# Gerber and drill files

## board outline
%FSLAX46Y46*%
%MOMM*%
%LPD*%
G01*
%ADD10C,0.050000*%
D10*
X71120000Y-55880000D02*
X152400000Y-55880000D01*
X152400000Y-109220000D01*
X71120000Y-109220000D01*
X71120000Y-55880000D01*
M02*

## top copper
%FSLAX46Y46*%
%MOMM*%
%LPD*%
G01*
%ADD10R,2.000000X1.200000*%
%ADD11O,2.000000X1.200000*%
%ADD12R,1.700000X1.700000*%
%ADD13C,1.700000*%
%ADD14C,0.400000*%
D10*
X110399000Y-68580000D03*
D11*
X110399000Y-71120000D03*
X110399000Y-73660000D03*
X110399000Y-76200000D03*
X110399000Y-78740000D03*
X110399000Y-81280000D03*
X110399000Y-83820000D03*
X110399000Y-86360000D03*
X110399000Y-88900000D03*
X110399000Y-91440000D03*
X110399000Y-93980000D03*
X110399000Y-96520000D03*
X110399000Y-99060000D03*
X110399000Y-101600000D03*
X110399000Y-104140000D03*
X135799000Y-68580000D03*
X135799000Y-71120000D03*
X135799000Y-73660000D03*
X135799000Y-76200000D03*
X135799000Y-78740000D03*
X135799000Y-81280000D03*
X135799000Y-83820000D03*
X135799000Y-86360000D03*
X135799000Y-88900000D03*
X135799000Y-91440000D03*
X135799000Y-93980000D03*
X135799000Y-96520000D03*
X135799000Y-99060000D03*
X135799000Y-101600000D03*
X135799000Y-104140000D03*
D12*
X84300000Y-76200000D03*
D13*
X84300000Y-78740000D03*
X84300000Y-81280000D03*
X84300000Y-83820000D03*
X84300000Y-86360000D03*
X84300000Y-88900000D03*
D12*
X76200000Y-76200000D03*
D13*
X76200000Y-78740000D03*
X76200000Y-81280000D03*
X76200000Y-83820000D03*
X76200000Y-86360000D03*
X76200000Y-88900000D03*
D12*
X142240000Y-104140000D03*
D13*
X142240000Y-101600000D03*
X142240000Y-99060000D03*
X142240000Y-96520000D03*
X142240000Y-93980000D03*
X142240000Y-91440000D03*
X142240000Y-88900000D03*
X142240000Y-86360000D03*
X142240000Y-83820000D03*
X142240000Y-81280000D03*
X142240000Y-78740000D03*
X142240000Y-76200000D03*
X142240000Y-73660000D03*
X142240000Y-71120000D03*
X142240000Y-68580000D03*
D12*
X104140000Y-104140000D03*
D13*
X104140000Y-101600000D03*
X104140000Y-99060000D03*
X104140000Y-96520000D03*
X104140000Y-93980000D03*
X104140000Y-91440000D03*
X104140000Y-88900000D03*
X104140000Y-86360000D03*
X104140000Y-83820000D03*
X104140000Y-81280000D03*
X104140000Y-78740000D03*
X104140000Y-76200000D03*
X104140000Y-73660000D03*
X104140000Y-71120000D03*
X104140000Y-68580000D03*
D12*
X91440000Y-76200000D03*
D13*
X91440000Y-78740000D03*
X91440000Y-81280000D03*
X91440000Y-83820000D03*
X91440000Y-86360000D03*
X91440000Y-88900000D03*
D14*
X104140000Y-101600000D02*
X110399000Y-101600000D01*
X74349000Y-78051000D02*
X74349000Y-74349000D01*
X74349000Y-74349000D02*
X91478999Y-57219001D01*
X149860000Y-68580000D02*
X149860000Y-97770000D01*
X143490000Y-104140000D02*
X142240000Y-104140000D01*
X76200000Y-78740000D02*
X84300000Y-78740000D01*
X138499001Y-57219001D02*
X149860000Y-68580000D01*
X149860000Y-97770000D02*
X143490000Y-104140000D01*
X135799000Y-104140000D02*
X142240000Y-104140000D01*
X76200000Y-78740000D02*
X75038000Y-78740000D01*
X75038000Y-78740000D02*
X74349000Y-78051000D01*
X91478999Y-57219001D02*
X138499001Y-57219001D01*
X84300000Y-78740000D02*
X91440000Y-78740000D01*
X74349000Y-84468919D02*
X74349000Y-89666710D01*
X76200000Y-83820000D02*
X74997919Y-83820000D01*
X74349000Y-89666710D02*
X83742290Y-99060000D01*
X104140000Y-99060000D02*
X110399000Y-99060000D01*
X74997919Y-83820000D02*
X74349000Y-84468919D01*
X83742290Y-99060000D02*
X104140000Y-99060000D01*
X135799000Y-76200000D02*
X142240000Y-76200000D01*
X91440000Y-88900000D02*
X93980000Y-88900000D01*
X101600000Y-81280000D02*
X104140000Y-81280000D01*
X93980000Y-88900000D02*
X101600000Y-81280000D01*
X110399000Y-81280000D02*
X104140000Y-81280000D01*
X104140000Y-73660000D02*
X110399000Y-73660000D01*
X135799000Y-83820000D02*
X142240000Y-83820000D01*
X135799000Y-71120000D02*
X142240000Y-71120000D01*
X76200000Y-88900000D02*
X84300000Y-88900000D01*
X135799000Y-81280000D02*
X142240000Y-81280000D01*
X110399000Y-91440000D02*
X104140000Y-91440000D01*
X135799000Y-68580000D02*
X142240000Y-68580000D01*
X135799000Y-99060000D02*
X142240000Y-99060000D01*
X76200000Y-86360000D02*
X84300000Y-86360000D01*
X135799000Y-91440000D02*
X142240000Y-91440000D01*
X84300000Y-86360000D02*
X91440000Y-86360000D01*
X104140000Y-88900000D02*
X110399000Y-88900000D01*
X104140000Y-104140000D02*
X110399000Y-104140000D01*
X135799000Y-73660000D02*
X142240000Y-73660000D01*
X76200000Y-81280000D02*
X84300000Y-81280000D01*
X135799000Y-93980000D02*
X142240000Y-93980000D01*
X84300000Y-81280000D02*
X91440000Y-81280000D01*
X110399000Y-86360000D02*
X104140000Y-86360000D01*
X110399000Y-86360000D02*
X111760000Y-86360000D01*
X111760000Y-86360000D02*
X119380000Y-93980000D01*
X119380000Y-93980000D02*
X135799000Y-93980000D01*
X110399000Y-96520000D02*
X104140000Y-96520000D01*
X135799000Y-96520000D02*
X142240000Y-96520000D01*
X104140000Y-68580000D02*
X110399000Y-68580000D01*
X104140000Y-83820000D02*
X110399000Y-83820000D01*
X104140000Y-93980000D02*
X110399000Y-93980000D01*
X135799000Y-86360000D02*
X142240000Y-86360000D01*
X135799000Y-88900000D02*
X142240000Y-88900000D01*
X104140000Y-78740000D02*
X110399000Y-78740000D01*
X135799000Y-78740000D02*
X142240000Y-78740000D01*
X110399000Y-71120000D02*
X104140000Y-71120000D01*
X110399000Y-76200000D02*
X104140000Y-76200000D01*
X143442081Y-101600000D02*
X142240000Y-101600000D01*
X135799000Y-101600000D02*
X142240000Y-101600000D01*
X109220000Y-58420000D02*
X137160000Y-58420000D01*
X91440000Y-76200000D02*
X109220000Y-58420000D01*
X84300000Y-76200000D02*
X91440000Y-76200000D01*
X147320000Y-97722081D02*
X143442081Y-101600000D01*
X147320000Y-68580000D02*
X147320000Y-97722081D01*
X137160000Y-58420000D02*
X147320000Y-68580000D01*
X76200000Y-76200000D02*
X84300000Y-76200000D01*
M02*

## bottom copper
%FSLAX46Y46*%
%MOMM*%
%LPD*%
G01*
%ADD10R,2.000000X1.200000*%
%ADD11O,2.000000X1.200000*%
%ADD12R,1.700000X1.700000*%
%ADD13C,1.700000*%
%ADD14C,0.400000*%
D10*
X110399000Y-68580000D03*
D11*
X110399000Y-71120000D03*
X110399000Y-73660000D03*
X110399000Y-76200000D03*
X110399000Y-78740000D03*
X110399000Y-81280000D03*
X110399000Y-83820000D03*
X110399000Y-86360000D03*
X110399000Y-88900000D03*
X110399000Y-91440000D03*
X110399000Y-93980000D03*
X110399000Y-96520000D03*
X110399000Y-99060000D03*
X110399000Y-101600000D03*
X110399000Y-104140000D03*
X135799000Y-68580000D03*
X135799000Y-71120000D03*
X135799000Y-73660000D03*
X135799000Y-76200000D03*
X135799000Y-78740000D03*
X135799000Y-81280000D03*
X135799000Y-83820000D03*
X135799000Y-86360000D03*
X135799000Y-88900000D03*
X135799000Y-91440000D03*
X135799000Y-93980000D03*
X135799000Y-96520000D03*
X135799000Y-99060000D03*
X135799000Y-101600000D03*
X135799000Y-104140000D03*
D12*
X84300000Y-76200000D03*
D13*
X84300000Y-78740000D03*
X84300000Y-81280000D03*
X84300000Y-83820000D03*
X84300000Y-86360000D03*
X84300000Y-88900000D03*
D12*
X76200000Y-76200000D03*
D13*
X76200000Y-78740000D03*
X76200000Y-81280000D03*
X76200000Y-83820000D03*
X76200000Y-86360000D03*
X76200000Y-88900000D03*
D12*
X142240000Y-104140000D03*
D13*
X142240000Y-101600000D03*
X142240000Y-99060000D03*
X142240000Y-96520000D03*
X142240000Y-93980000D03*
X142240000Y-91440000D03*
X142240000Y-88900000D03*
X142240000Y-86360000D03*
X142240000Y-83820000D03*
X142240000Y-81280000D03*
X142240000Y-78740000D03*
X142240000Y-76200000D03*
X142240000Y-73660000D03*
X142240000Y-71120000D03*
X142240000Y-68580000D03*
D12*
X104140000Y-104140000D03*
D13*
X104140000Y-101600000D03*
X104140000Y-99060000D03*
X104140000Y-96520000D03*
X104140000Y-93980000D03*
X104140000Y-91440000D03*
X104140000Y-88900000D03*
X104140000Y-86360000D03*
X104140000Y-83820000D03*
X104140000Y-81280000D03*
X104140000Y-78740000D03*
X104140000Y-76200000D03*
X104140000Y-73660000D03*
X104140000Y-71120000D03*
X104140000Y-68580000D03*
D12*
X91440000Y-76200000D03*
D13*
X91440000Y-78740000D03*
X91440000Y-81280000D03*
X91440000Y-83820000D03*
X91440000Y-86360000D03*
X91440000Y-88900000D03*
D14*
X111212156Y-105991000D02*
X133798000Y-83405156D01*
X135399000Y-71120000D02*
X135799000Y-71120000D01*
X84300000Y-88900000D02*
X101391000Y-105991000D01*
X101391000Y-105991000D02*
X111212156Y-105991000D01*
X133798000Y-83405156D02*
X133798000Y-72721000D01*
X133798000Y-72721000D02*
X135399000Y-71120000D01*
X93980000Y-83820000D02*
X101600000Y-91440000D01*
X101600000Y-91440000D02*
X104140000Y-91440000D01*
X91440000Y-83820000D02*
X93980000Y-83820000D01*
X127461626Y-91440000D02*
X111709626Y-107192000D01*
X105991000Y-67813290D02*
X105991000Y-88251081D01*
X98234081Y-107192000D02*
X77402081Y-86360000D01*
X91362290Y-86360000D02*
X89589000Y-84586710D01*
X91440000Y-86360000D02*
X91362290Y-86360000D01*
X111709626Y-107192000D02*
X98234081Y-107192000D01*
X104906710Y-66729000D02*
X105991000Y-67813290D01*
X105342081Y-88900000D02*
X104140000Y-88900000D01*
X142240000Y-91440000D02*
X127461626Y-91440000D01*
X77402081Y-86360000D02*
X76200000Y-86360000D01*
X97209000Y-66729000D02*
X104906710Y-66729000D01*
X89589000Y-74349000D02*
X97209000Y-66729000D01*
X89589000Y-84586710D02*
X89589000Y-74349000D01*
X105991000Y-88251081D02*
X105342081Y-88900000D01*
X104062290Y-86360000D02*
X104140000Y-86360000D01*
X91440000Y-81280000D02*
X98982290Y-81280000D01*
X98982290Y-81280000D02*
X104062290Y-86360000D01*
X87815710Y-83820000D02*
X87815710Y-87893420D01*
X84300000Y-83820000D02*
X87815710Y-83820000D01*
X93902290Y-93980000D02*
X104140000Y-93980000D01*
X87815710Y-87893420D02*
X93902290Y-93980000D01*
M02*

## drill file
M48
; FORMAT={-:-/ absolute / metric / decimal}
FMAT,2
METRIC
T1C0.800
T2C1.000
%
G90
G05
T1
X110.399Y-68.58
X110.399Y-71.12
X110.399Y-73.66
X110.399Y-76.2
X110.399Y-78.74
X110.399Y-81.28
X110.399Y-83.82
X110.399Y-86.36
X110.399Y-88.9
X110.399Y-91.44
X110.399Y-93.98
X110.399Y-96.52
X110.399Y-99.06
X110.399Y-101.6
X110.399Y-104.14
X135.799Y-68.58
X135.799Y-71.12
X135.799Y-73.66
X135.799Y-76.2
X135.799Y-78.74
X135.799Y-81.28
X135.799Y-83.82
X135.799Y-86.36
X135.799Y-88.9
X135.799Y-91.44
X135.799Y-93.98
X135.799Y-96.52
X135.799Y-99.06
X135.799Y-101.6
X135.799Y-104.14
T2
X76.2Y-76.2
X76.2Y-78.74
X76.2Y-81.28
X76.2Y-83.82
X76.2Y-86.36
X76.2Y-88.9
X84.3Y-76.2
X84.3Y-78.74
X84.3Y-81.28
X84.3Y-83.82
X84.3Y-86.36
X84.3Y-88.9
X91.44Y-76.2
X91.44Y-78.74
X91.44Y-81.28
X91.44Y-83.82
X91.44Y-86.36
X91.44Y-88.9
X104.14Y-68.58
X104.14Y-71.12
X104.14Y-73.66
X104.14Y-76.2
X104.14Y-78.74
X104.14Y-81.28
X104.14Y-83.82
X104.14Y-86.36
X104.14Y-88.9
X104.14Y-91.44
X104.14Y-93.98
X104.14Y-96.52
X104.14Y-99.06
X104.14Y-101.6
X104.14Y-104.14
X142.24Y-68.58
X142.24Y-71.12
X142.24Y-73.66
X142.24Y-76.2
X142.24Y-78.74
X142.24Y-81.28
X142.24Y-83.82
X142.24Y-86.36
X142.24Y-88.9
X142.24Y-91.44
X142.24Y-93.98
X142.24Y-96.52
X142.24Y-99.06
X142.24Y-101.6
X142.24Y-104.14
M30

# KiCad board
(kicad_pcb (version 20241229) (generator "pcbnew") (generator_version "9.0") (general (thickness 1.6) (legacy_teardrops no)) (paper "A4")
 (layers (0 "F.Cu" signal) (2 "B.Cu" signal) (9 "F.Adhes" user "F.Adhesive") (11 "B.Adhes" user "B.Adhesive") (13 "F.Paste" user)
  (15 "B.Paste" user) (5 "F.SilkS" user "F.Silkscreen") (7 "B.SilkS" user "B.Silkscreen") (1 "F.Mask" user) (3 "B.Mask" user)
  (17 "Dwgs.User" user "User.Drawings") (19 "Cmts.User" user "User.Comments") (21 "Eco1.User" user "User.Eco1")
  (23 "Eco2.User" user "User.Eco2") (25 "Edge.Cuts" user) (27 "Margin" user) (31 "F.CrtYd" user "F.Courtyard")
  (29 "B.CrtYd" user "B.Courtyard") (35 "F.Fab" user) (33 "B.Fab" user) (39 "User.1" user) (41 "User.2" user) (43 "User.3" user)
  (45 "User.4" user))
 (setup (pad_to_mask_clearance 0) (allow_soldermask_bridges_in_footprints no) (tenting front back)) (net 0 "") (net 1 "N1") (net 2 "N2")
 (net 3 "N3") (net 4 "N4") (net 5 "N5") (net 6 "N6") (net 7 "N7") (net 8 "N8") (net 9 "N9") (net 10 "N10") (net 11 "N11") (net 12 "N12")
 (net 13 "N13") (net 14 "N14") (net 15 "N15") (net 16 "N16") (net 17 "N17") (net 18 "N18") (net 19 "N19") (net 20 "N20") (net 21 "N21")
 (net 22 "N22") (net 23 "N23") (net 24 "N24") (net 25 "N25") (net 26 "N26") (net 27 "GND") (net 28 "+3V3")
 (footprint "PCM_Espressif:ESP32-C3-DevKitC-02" (layer "F.Cu") (at 110.399 68.58)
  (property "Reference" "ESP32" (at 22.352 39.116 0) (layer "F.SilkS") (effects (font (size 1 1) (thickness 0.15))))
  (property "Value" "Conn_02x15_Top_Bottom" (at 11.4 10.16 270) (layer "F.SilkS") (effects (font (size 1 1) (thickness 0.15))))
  (pad "1" thru_hole rect (at 0 0 270) (size 1.2 2) (drill 0.8) (layers "*.Cu" "*.Mask") (remove_unused_layers no) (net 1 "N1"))
  (pad "2" thru_hole oval (at 0 2.54 270) (size 1.2 2) (drill 0.8) (layers "*.Cu" "*.Mask") (remove_unused_layers no) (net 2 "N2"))
  (pad "3" thru_hole oval (at 0 5.08 270) (size 1.2 2) (drill 0.8) (layers "*.Cu" "*.Mask") (remove_unused_layers no) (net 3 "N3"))
  (pad "4" thru_hole oval (at 0 7.62 270) (size 1.2 2) (drill 0.8) (layers "*.Cu" "*.Mask") (remove_unused_layers no) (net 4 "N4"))
  (pad "5" thru_hole oval (at 0 10.16 270) (size 1.2 2) (drill 0.8) (layers "*.Cu" "*.Mask") (remove_unused_layers no) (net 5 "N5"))
  (pad "6" thru_hole oval (at 0 12.7 270) (size 1.2 2) (drill 0.8) (layers "*.Cu" "*.Mask") (remove_unused_layers no) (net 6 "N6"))
  (pad "7" thru_hole oval (at 0 15.24 270) (size 1.2 2) (drill 0.8) (layers "*.Cu" "*.Mask") (remove_unused_layers no) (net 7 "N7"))
  (pad "8" thru_hole oval (at 0 17.78 270) (size 1.2 2) (drill 0.8) (layers "*.Cu" "*.Mask") (remove_unused_layers no) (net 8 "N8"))
  (pad "9" thru_hole oval (at 0 20.32 270) (size 1.2 2) (drill 0.8) (layers "*.Cu" "*.Mask") (remove_unused_layers no) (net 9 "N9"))
  (pad "10" thru_hole oval (at 0 22.86 270) (size 1.2 2) (drill 0.8) (layers "*.Cu" "*.Mask") (remove_unused_layers no) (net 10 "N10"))
  (pad "11" thru_hole oval (at 0 25.4 270) (size 1.2 2) (drill 0.8) (layers "*.Cu" "*.Mask") (remove_unused_layers no) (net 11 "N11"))
  (pad "12" thru_hole oval (at 0 27.94 270) (size 1.2 2) (drill 0.8) (layers "*.Cu" "*.Mask") (remove_unused_layers no) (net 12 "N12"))
  (pad "13" thru_hole oval (at 0 30.48 270) (size 1.2 2) (drill 0.8) (layers "*.Cu" "*.Mask") (remove_unused_layers no) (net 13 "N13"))
  (pad "14" thru_hole oval (at 0 33.02 270) (size 1.2 2) (drill 0.8) (layers "*.Cu" "*.Mask") (remove_unused_layers no) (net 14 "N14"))
  (pad "15" thru_hole oval (at 0 35.56 270) (size 1.2 2) (drill 0.8) (layers "*.Cu" "*.Mask") (remove_unused_layers no) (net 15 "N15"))
  (pad "16" thru_hole oval (at 25.4 0 90) (size 1.2 2) (drill 0.8) (layers "*.Cu" "*.Mask") (remove_unused_layers no) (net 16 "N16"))
  (pad "17" thru_hole oval (at 25.4 2.54 90) (size 1.2 2) (drill 0.8) (layers "*.Cu" "*.Mask") (remove_unused_layers no) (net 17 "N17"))
  (pad "18" thru_hole oval (at 25.4 5.08 90) (size 1.2 2) (drill 0.8) (layers "*.Cu" "*.Mask") (remove_unused_layers no) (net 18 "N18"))
  (pad "19" thru_hole oval (at 25.4 7.62 90) (size 1.2 2) (drill 0.8) (layers "*.Cu" "*.Mask") (remove_unused_layers no) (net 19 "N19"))
  (pad "20" thru_hole oval (at 25.4 10.16 90) (size 1.2 2) (drill 0.8) (layers "*.Cu" "*.Mask") (remove_unused_layers no) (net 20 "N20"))
  (pad "21" thru_hole oval (at 25.4 12.7 90) (size 1.2 2) (drill 0.8) (layers "*.Cu" "*.Mask") (remove_unused_layers no) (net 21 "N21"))
  (pad "22" thru_hole oval (at 25.4 15.24 90) (size 1.2 2) (drill 0.8) (layers "*.Cu" "*.Mask") (remove_unused_layers no) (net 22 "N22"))
  (pad "23" thru_hole oval (at 25.4 17.78 90) (size 1.2 2) (drill 0.8) (layers "*.Cu" "*.Mask") (remove_unused_layers no) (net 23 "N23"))
  (pad "24" thru_hole oval (at 25.4 20.32 90) (size 1.2 2) (drill 0.8) (layers "*.Cu" "*.Mask") (remove_unused_layers no) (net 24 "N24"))
  (pad "25" thru_hole oval (at 25.4 22.86 90) (size 1.2 2) (drill 0.8) (layers "*.Cu" "*.Mask") (remove_unused_layers no) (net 9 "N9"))
  (pad "26" thru_hole oval (at 25.4 25.4 90) (size 1.2 2) (drill 0.8) (layers "*.Cu" "*.Mask") (remove_unused_layers no) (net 8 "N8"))
  (pad "27" thru_hole oval (at 25.4 27.94 90) (size 1.2 2) (drill 0.8) (layers "*.Cu" "*.Mask") (remove_unused_layers no) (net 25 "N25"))
  (pad "28" thru_hole oval (at 25.4 30.48 90) (size 1.2 2) (drill 0.8) (layers "*.Cu" "*.Mask") (remove_unused_layers no) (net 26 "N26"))
  (pad "29" thru_hole oval (at 25.4 33.02 90) (size 1.2 2) (drill 0.8) (layers "*.Cu" "*.Mask") (remove_unused_layers no) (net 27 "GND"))
  (pad "30" thru_hole oval (at 25.4 35.56 90) (size 1.2 2) (drill 0.8) (layers "*.Cu" "*.Mask") (remove_unused_layers no) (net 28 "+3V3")))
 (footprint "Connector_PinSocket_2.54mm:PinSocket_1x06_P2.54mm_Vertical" (layer "F.Cu") (at 84.3 76.2)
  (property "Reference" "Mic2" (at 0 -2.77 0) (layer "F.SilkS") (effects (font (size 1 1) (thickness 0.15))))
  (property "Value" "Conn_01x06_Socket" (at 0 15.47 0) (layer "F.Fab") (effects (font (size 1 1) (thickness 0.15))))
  (pad "1" thru_hole rect (at 0 0) (size 1.7 1.7) (drill 1) (layers "*.Cu" "*.Mask") (remove_unused_layers no) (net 27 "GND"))
  (pad "2" thru_hole circle (at 0 2.54) (size 1.7 1.7) (drill 1) (layers "*.Cu" "*.Mask") (remove_unused_layers no) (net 28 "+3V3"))
  (pad "3" thru_hole circle (at 0 5.08) (size 1.7 1.7) (drill 1) (layers "*.Cu" "*.Mask") (remove_unused_layers no) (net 8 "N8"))
  (pad "4" thru_hole circle (at 0 7.62) (size 1.7 1.7) (drill 1) (layers "*.Cu" "*.Mask") (remove_unused_layers no) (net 11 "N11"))
  (pad "5" thru_hole circle (at 0 10.16) (size 1.7 1.7) (drill 1) (layers "*.Cu" "*.Mask") (remove_unused_layers no) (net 9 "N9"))
  (pad "6" thru_hole circle (at 0 12.7) (size 1.7 1.7) (drill 1) (layers "*.Cu" "*.Mask") (remove_unused_layers no) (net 17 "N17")))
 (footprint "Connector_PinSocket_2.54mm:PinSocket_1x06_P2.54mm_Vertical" (layer "F.Cu") (at 76.2 76.2)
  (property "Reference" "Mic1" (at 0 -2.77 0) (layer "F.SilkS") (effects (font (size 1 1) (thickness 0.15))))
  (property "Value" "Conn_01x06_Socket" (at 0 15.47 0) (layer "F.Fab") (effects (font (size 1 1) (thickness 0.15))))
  (pad "1" thru_hole rect (at 0 0) (size 1.7 1.7) (drill 1) (layers "*.Cu" "*.Mask") (remove_unused_layers no) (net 27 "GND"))
  (pad "2" thru_hole circle (at 0 2.54) (size 1.7 1.7) (drill 1) (layers "*.Cu" "*.Mask") (remove_unused_layers no) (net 28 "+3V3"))
  (pad "3" thru_hole circle (at 0 5.08) (size 1.7 1.7) (drill 1) (layers "*.Cu" "*.Mask") (remove_unused_layers no) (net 8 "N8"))
  (pad "4" thru_hole circle (at 0 7.62) (size 1.7 1.7) (drill 1) (layers "*.Cu" "*.Mask") (remove_unused_layers no) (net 13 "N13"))
  (pad "5" thru_hole circle (at 0 10.16) (size 1.7 1.7) (drill 1) (layers "*.Cu" "*.Mask") (remove_unused_layers no) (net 9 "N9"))
  (pad "6" thru_hole circle (at 0 12.7) (size 1.7 1.7) (drill 1) (layers "*.Cu" "*.Mask") (remove_unused_layers no) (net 17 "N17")))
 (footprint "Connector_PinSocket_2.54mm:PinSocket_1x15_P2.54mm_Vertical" (layer "F.Cu") (at 142.24 104.14 180)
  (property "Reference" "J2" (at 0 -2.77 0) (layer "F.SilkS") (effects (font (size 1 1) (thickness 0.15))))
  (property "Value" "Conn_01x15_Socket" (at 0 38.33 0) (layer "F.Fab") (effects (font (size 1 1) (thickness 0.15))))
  (pad "1" thru_hole rect (at 0 0 180) (size 1.7 1.7) (drill 1) (layers "*.Cu" "*.Mask") (remove_unused_layers no) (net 28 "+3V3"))
  (pad "2" thru_hole circle (at 0 2.54 180) (size 1.7 1.7) (drill 1) (layers "*.Cu" "*.Mask") (remove_unused_layers no) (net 27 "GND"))
  (pad "3" thru_hole circle (at 0 5.08 180) (size 1.7 1.7) (drill 1) (layers "*.Cu" "*.Mask") (remove_unused_layers no) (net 26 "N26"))
  (pad "4" thru_hole circle (at 0 7.62 180) (size 1.7 1.7) (drill 1) (layers "*.Cu" "*.Mask") (remove_unused_layers no) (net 25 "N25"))
  (pad "5" thru_hole circle (at 0 10.16 180) (size 1.7 1.7) (drill 1) (layers "*.Cu" "*.Mask") (remove_unused_layers no) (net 8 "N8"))
  (pad "6" thru_hole circle (at 0 12.7 180) (size 1.7 1.7) (drill 1) (layers "*.Cu" "*.Mask") (remove_unused_layers no) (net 9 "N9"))
  (pad "7" thru_hole circle (at 0 15.24 180) (size 1.7 1.7) (drill 1) (layers "*.Cu" "*.Mask") (remove_unused_layers no) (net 24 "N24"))
  (pad "8" thru_hole circle (at 0 17.78 180) (size 1.7 1.7) (drill 1) (layers "*.Cu" "*.Mask") (remove_unused_layers no) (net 23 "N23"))
  (pad "9" thru_hole circle (at 0 20.32 180) (size 1.7 1.7) (drill 1) (layers "*.Cu" "*.Mask") (remove_unused_layers no) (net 22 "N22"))
  (pad "10" thru_hole circle (at 0 22.86 180) (size 1.7 1.7) (drill 1) (layers "*.Cu" "*.Mask") (remove_unused_layers no) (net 21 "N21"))
  (pad "11" thru_hole circle (at 0 25.4 180) (size 1.7 1.7) (drill 1) (layers "*.Cu" "*.Mask") (remove_unused_layers no) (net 20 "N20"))
  (pad "12" thru_hole circle (at 0 27.94 180) (size 1.7 1.7) (drill 1) (layers "*.Cu" "*.Mask") (remove_unused_layers no) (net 19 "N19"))
  (pad "13" thru_hole circle (at 0 30.48 180) (size 1.7 1.7) (drill 1) (layers "*.Cu" "*.Mask") (remove_unused_layers no) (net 18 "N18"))
  (pad "14" thru_hole circle (at 0 33.02 180) (size 1.7 1.7) (drill 1) (layers "*.Cu" "*.Mask") (remove_unused_layers no) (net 17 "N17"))
  (pad "15" thru_hole circle (at 0 35.56 180) (size 1.7 1.7) (drill 1) (layers "*.Cu" "*.Mask") (remove_unused_layers no) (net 16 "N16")))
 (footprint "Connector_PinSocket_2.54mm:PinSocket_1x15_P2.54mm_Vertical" (layer "F.Cu") (at 104.14 104.14 180)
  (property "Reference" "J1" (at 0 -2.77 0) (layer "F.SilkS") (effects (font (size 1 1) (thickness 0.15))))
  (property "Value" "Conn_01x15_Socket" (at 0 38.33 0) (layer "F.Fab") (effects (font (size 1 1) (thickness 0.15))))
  (pad "1" thru_hole rect (at 0 0 180) (size 1.7 1.7) (drill 1) (layers "*.Cu" "*.Mask") (remove_unused_layers no) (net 15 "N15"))
  (pad "2" thru_hole circle (at 0 2.54 180) (size 1.7 1.7) (drill 1) (layers "*.Cu" "*.Mask") (remove_unused_layers no) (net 14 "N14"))
  (pad "3" thru_hole circle (at 0 5.08 180) (size 1.7 1.7) (drill 1) (layers "*.Cu" "*.Mask") (remove_unused_layers no) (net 13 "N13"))
  (pad "4" thru_hole circle (at 0 7.62 180) (size 1.7 1.7) (drill 1) (layers "*.Cu" "*.Mask") (remove_unused_layers no) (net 12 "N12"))
  (pad "5" thru_hole circle (at 0 10.16 180) (size 1.7 1.7) (drill 1) (layers "*.Cu" "*.Mask") (remove_unused_layers no) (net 11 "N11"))
  (pad "6" thru_hole circle (at 0 12.7 180) (size 1.7 1.7) (drill 1) (layers "*.Cu" "*.Mask") (remove_unused_layers no) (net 10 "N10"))
  (pad "7" thru_hole circle (at 0 15.24 180) (size 1.7 1.7) (drill 1) (layers "*.Cu" "*.Mask") (remove_unused_layers no) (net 9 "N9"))
  (pad "8" thru_hole circle (at 0 17.78 180) (size 1.7 1.7) (drill 1) (layers "*.Cu" "*.Mask") (remove_unused_layers no) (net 8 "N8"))
  (pad "9" thru_hole circle (at 0 20.32 180) (size 1.7 1.7) (drill 1) (layers "*.Cu" "*.Mask") (remove_unused_layers no) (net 7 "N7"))
  (pad "10" thru_hole circle (at 0 22.86 180) (size 1.7 1.7) (drill 1) (layers "*.Cu" "*.Mask") (remove_unused_layers no) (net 6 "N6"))
  (pad "11" thru_hole circle (at 0 25.4 180) (size 1.7 1.7) (drill 1) (layers "*.Cu" "*.Mask") (remove_unused_layers no) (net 5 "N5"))
  (pad "12" thru_hole circle (at 0 27.94 180) (size 1.7 1.7) (drill 1) (layers "*.Cu" "*.Mask") (remove_unused_layers no) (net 4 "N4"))
  (pad "13" thru_hole circle (at 0 30.48 180) (size 1.7 1.7) (drill 1) (layers "*.Cu" "*.Mask") (remove_unused_layers no) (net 3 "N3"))
  (pad "14" thru_hole circle (at 0 33.02 180) (size 1.7 1.7) (drill 1) (layers "*.Cu" "*.Mask") (remove_unused_layers no) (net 2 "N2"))
  (pad "15" thru_hole circle (at 0 35.56 180) (size 1.7 1.7) (drill 1) (layers "*.Cu" "*.Mask") (remove_unused_layers no) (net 1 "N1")))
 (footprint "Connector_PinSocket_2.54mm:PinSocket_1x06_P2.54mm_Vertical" (layer "F.Cu") (at 91.44 76.2)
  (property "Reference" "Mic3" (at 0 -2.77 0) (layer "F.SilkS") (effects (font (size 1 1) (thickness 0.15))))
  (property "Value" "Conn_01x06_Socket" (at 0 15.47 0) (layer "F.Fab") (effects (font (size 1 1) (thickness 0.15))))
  (pad "1" thru_hole rect (at 0 0) (size 1.7 1.7) (drill 1) (layers "*.Cu" "*.Mask") (remove_unused_layers no) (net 27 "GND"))
  (pad "2" thru_hole circle (at 0 2.54) (size 1.7 1.7) (drill 1) (layers "*.Cu" "*.Mask") (remove_unused_layers no) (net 28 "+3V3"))
  (pad "3" thru_hole circle (at 0 5.08) (size 1.7 1.7) (drill 1) (layers "*.Cu" "*.Mask") (remove_unused_layers no) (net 8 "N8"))
  (pad "4" thru_hole circle (at 0 7.62) (size 1.7 1.7) (drill 1) (layers "*.Cu" "*.Mask") (remove_unused_layers no) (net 10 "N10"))
  (pad "5" thru_hole circle (at 0 10.16) (size 1.7 1.7) (drill 1) (layers "*.Cu" "*.Mask") (remove_unused_layers no) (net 9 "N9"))
  (pad "6" thru_hole circle (at 0 12.7) (size 1.7 1.7) (drill 1) (layers "*.Cu" "*.Mask") (remove_unused_layers no) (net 6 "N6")))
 (gr_rect (start 71.12 55.88) (end 152.4 109.22) (stroke (width 0.05) (type default)) (fill no) (layer "Edge.Cuts"))
 (segment (start 104.14 101.6) (end 110.399 101.6) (width 0.4) (layer "F.Cu") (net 14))
 (segment (start 74.349 78.051) (end 74.349 74.349) (width 0.4) (layer "F.Cu") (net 28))
 (segment (start 74.349 74.349) (end 91.478999 57.219001) (width 0.4) (layer "F.Cu") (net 28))
 (segment (start 149.86 68.58) (end 149.86 97.77) (width 0.4) (layer "F.Cu") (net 28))
 (segment (start 143.49 104.14) (end 142.24 104.14) (width 0.4) (layer "F.Cu") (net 28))
 (segment (start 76.2 78.74) (end 84.3 78.74) (width 0.4) (layer "F.Cu") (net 28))
 (segment (start 138.499001 57.219001) (end 149.86 68.58) (width 0.4) (layer "F.Cu") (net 28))
 (segment (start 149.86 97.77) (end 143.49 104.14) (width 0.4) (layer "F.Cu") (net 28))
 (segment (start 135.799 104.14) (end 142.24 104.14) (width 0.4) (layer "F.Cu") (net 28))
 (segment (start 76.2 78.74) (end 75.038 78.74) (width 0.4) (layer "F.Cu") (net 28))
 (segment (start 75.038 78.74) (end 74.349 78.051) (width 0.4) (layer "F.Cu") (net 28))
 (segment (start 91.478999 57.219001) (end 138.499001 57.219001) (width 0.4) (layer "F.Cu") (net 28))
 (segment (start 84.3 78.74) (end 91.44 78.74) (width 0.4) (layer "F.Cu") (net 28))
 (segment (start 74.349 84.468919) (end 74.349 89.66671) (width 0.4) (layer "F.Cu") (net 13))
 (segment (start 76.2 83.82) (end 74.997919 83.82) (width 0.4) (layer "F.Cu") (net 13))
 (segment (start 74.349 89.66671) (end 83.74229 99.06) (width 0.4) (layer "F.Cu") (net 13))
 (segment (start 104.14 99.06) (end 110.399 99.06) (width 0.4) (layer "F.Cu") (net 13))
 (segment (start 74.997919 83.82) (end 74.349 84.468919) (width 0.4) (layer "F.Cu") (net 13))
 (segment (start 83.74229 99.06) (end 104.14 99.06) (width 0.4) (layer "F.Cu") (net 13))
 (segment (start 135.799 76.2) (end 142.24 76.2) (width 0.4) (layer "F.Cu") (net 19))
 (segment (start 91.44 88.9) (end 93.98 88.9) (width 0.4) (layer "F.Cu") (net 6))
 (segment (start 101.6 81.28) (end 104.14 81.28) (width 0.4) (layer "F.Cu") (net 6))
 (segment (start 93.98 88.9) (end 101.6 81.28) (width 0.4) (layer "F.Cu") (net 6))
 (segment (start 110.399 81.28) (end 104.14 81.28) (width 0.4) (layer "F.Cu") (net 6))
 (segment (start 104.14 73.66) (end 110.399 73.66) (width 0.4) (layer "F.Cu") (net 3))
 (segment (start 135.799 83.82) (end 142.24 83.82) (width 0.4) (layer "F.Cu") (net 22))
 (segment (start 135.799 71.12) (end 142.24 71.12) (width 0.4) (layer "F.Cu") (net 17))
 (segment (start 76.2 88.9) (end 84.3 88.9) (width 0.4) (layer "F.Cu") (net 17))
 (segment (start 111.212156 105.991) (end 133.798 83.405156) (width 0.4) (layer "B.Cu") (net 17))
 (segment (start 135.399 71.12) (end 135.799 71.12) (width 0.4) (layer "B.Cu") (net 17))
 (segment (start 84.3 88.9) (end 101.391 105.991) (width 0.4) (layer "B.Cu") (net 17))
 (segment (start 101.391 105.991) (end 111.212156 105.991) (width 0.4) (layer "B.Cu") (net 17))
 (segment (start 133.798 83.405156) (end 133.798 72.721) (width 0.4) (layer "B.Cu") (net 17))
 (segment (start 133.798 72.721) (end 135.399 71.12) (width 0.4) (layer "B.Cu") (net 17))
 (segment (start 135.799 81.28) (end 142.24 81.28) (width 0.4) (layer "F.Cu") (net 21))
 (segment (start 110.399 91.44) (end 104.14 91.44) (width 0.4) (layer "F.Cu") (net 10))
 (segment (start 93.98 83.82) (end 101.6 91.44) (width 0.4) (layer "B.Cu") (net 10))
 (segment (start 101.6 91.44) (end 104.14 91.44) (width 0.4) (layer "B.Cu") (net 10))
 (segment (start 91.44 83.82) (end 93.98 83.82) (width 0.4) (layer "B.Cu") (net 10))
 (segment (start 135.799 68.58) (end 142.24 68.58) (width 0.4) (layer "F.Cu") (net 16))
 (segment (start 135.799 99.06) (end 142.24 99.06) (width 0.4) (layer "F.Cu") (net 26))
 (segment (start 76.2 86.36) (end 84.3 86.36) (width 0.4) (layer "F.Cu") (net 9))
 (segment (start 135.799 91.44) (end 142.24 91.44) (width 0.4) (layer "F.Cu") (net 9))
 (segment (start 84.3 86.36) (end 91.44 86.36) (width 0.4) (layer "F.Cu") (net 9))
 (segment (start 104.14 88.9) (end 110.399 88.9) (width 0.4) (layer "F.Cu") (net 9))
 (segment (start 127.461626 91.44) (end 111.709626 107.192) (width 0.4) (layer "B.Cu") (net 9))
 (segment (start 105.991 67.81329) (end 105.991 88.251081) (width 0.4) (layer "B.Cu") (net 9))
 (segment (start 98.234081 107.192) (end 77.402081 86.36) (width 0.4) (layer "B.Cu") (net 9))
 (segment (start 91.36229 86.36) (end 89.589 84.58671) (width 0.4) (layer "B.Cu") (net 9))
 (segment (start 91.44 86.36) (end 91.36229 86.36) (width 0.4) (layer "B.Cu") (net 9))
 (segment (start 111.709626 107.192) (end 98.234081 107.192) (width 0.4) (layer "B.Cu") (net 9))
 (segment (start 104.90671 66.729) (end 105.991 67.81329) (width 0.4) (layer "B.Cu") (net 9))
 (segment (start 105.342081 88.9) (end 104.14 88.9) (width 0.4) (layer "B.Cu") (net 9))
 (segment (start 142.24 91.44) (end 127.461626 91.44) (width 0.4) (layer "B.Cu") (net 9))
 (segment (start 77.402081 86.36) (end 76.2 86.36) (width 0.4) (layer "B.Cu") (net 9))
 (segment (start 97.209 66.729) (end 104.90671 66.729) (width 0.4) (layer "B.Cu") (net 9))
 (segment (start 89.589 74.349) (end 97.209 66.729) (width 0.4) (layer "B.Cu") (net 9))
 (segment (start 89.589 84.58671) (end 89.589 74.349) (width 0.4) (layer "B.Cu") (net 9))
 (segment (start 105.991 88.251081) (end 105.342081 88.9) (width 0.4) (layer "B.Cu") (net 9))
 (segment (start 104.14 104.14) (end 110.399 104.14) (width 0.4) (layer "F.Cu") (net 15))
 (segment (start 135.799 73.66) (end 142.24 73.66) (width 0.4) (layer "F.Cu") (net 18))
 (segment (start 76.2 81.28) (end 84.3 81.28) (width 0.4) (layer "F.Cu") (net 8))
 (segment (start 135.799 93.98) (end 142.24 93.98) (width 0.4) (layer "F.Cu") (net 8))
 (segment (start 84.3 81.28) (end 91.44 81.28) (width 0.4) (layer "F.Cu") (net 8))
 (segment (start 110.399 86.36) (end 104.14 86.36) (width 0.4) (layer "F.Cu") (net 8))
 (segment (start 110.399 86.36) (end 111.76 86.36) (width 0.4) (layer "F.Cu") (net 8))
 (segment (start 111.76 86.36) (end 119.38 93.98) (width 0.4) (layer "F.Cu") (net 8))
 (segment (start 119.38 93.98) (end 135.799 93.98) (width 0.4) (layer "F.Cu") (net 8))
 (segment (start 104.06229 86.36) (end 104.14 86.36) (width 0.4) (layer "B.Cu") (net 8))
 (segment (start 91.44 81.28) (end 98.98229 81.28) (width 0.4) (layer "B.Cu") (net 8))
 (segment (start 98.98229 81.28) (end 104.06229 86.36) (width 0.4) (layer "B.Cu") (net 8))
 (segment (start 110.399 96.52) (end 104.14 96.52) (width 0.4) (layer "F.Cu") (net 12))
 (segment (start 135.799 96.52) (end 142.24 96.52) (width 0.4) (layer "F.Cu") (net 25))
 (segment (start 104.14 68.58) (end 110.399 68.58) (width 0.4) (layer "F.Cu") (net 1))
 (segment (start 104.14 83.82) (end 110.399 83.82) (width 0.4) (layer "F.Cu") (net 7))
 (segment (start 104.14 93.98) (end 110.399 93.98) (width 0.4) (layer "F.Cu") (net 11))
 (segment (start 87.81571 83.82) (end 87.81571 87.89342) (width 0.4) (layer "B.Cu") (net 11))
 (segment (start 84.3 83.82) (end 87.81571 83.82) (width 0.4) (layer "B.Cu") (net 11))
 (segment (start 93.90229 93.98) (end 104.14 93.98) (width 0.4) (layer "B.Cu") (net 11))
 (segment (start 87.81571 87.89342) (end 93.90229 93.98) (width 0.4) (layer "B.Cu") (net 11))
 (segment (start 135.799 86.36) (end 142.24 86.36) (width 0.4) (layer "F.Cu") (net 23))
 (segment (start 135.799 88.9) (end 142.24 88.9) (width 0.4) (layer "F.Cu") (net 24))
 (segment (start 104.14 78.74) (end 110.399 78.74) (width 0.4) (layer "F.Cu") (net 5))
 (segment (start 135.799 78.74) (end 142.24 78.74) (width 0.4) (layer "F.Cu") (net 20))
 (segment (start 110.399 71.12) (end 104.14 71.12) (width 0.4) (layer "F.Cu") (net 2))
 (segment (start 110.399 76.2) (end 104.14 76.2) (width 0.4) (layer "F.Cu") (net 4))
 (segment (start 143.442081 101.6) (end 142.24 101.6) (width 0.4) (layer "F.Cu") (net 27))
 (segment (start 135.799 101.6) (end 142.24 101.6) (width 0.4) (layer "F.Cu") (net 27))
 (segment (start 109.22 58.42) (end 137.16 58.42) (width 0.4) (layer "F.Cu") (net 27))
 (segment (start 91.44 76.2) (end 109.22 58.42) (width 0.4) (layer "F.Cu") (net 27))
 (segment (start 84.3 76.2) (end 91.44 76.2) (width 0.4) (layer "F.Cu") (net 27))
 (segment (start 147.32 97.722081) (end 143.442081 101.6) (width 0.4) (layer "F.Cu") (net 27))
 (segment (start 147.32 68.58) (end 147.32 97.722081) (width 0.4) (layer "F.Cu") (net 27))
 (segment (start 137.16 58.42) (end 147.32 68.58) (width 0.4) (layer "F.Cu") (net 27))
 (segment (start 76.2 76.2) (end 84.3 76.2) (width 0.4) (layer "F.Cu") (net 27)))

